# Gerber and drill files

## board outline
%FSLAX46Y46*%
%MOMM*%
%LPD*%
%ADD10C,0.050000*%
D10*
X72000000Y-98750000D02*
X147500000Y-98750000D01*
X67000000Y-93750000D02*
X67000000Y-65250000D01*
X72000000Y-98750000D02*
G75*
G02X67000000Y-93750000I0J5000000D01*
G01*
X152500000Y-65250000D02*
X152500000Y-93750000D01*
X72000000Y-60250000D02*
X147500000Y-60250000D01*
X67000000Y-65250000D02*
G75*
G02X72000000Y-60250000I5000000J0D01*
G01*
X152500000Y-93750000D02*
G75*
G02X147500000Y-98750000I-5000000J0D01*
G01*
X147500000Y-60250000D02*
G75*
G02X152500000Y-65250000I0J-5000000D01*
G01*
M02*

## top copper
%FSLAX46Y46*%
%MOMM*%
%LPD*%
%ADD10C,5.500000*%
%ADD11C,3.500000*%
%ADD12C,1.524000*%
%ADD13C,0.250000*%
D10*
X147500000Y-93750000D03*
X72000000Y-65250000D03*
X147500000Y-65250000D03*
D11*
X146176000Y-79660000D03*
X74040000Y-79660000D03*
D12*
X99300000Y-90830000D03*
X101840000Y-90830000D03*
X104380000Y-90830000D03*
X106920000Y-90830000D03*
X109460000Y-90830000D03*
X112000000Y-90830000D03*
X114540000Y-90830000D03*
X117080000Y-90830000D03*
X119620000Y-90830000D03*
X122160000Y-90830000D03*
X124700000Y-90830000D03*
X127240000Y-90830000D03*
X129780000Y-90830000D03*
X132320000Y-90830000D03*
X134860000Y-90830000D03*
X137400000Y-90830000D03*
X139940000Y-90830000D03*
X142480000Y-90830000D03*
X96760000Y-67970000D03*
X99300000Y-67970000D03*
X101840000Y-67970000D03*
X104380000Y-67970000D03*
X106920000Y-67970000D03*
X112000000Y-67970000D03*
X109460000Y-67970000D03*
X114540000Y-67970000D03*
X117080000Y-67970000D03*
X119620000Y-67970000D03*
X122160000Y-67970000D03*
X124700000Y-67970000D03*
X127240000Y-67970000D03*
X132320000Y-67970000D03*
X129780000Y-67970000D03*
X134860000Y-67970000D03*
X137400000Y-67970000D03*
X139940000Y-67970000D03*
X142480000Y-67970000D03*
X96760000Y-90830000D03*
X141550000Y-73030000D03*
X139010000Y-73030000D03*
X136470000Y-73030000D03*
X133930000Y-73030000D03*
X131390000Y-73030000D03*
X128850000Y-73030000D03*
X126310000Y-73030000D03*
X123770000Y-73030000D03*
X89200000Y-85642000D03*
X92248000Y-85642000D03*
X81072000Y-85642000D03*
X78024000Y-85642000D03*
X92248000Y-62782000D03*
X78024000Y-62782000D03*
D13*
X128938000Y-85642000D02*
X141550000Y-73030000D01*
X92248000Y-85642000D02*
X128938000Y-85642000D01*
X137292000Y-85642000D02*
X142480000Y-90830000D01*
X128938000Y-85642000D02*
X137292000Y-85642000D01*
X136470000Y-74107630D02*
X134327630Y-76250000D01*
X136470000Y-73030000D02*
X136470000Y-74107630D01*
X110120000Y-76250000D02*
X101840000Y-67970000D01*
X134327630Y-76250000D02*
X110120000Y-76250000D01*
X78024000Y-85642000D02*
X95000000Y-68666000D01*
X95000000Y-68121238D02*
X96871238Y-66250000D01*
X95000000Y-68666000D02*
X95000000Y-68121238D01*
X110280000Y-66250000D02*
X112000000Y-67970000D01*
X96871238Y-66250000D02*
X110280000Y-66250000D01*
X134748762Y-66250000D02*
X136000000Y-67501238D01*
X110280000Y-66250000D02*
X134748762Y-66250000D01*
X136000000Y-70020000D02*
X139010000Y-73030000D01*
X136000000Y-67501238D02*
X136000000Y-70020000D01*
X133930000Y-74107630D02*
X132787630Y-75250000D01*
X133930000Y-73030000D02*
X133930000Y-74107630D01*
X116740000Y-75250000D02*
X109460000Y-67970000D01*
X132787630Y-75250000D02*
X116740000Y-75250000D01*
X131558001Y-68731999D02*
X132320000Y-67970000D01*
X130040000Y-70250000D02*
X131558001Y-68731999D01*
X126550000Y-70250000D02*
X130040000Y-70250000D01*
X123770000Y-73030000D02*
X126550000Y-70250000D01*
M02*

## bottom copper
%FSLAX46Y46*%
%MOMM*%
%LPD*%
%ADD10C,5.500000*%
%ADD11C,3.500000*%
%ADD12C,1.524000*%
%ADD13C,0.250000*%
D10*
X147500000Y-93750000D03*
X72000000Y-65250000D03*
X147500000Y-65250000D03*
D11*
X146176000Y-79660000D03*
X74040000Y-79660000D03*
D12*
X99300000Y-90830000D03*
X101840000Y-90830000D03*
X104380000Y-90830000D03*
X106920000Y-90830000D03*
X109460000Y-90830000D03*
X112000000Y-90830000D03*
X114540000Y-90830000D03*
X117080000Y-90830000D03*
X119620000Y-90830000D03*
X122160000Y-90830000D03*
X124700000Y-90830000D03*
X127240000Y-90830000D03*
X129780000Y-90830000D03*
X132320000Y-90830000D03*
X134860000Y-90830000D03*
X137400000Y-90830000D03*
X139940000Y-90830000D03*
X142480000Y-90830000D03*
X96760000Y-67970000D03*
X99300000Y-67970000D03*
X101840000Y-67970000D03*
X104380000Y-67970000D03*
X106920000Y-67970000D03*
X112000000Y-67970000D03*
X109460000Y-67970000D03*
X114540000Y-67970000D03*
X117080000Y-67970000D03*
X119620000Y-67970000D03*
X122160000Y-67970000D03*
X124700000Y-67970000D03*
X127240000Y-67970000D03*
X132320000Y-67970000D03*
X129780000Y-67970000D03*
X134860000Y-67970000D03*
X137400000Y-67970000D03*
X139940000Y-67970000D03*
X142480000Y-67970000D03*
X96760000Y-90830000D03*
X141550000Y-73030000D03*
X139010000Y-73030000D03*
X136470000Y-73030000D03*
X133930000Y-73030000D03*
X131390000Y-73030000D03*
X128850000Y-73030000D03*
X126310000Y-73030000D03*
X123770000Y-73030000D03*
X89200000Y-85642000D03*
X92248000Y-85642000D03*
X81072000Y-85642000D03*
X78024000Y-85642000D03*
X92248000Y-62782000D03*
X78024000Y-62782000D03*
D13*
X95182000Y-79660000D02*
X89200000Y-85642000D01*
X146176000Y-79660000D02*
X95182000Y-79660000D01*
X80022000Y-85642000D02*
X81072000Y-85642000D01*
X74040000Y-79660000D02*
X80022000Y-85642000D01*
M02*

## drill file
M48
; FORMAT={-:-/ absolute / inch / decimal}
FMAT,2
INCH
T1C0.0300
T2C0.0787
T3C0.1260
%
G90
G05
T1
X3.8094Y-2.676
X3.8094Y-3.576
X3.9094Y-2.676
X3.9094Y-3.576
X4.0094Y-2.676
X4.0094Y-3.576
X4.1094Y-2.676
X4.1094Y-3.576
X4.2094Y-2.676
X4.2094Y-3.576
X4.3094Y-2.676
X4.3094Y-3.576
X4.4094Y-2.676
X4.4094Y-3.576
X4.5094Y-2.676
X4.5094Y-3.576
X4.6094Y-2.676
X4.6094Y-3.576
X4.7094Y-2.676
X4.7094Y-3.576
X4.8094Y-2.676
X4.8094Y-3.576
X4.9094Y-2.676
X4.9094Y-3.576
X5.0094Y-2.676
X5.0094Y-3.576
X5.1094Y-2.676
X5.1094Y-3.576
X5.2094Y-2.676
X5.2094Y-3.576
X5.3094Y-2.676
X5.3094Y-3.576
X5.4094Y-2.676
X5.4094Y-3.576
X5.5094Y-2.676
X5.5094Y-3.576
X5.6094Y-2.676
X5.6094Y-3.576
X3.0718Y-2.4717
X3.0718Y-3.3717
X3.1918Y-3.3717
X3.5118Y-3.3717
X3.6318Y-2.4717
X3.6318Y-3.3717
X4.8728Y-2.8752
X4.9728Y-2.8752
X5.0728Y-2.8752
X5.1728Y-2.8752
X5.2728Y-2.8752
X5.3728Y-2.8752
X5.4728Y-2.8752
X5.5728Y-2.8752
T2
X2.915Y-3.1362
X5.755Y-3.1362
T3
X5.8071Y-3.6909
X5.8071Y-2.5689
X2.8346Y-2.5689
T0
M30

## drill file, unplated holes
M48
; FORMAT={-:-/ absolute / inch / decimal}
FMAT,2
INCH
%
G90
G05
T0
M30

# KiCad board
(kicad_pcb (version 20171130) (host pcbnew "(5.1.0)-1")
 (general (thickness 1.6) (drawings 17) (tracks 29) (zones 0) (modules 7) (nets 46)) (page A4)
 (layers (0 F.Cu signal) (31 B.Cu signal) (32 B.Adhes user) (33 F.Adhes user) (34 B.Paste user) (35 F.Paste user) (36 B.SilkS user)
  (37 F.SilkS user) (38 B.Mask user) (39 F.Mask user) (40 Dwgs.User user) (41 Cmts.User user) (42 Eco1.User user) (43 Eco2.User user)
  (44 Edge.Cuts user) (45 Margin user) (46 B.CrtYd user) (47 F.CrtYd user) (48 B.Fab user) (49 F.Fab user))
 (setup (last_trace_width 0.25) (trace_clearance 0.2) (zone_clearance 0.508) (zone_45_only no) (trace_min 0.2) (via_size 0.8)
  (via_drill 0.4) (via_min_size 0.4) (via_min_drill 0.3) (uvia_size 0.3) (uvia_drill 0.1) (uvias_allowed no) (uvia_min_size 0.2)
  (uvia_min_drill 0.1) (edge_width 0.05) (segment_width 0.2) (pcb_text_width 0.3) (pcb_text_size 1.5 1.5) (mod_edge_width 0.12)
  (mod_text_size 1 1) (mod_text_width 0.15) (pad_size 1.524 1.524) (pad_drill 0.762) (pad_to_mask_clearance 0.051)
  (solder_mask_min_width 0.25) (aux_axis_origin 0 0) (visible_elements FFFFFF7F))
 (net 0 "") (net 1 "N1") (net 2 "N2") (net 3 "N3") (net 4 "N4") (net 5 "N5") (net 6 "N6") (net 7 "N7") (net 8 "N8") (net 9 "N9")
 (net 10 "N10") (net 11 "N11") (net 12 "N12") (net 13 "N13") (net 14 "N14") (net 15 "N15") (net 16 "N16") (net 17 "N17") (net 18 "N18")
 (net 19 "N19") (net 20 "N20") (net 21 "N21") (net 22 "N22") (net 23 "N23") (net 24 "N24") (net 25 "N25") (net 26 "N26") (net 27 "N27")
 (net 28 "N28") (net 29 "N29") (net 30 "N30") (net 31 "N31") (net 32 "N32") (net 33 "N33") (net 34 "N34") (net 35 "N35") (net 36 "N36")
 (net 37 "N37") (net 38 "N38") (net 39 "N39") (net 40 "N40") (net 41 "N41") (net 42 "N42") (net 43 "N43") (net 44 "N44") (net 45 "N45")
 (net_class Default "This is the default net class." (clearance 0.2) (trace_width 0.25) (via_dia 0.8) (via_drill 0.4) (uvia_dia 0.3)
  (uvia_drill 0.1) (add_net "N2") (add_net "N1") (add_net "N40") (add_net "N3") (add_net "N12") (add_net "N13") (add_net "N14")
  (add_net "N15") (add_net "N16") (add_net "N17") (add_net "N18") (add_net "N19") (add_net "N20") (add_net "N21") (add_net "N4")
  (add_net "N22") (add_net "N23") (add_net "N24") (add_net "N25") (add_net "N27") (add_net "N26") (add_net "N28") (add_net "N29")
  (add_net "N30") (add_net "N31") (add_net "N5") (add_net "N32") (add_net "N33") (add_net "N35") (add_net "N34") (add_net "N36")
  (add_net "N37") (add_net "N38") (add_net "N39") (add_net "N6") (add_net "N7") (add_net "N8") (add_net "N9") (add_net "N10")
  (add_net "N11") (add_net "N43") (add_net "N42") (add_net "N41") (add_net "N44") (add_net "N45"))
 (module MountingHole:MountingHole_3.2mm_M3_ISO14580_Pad (layer F.Cu) (at 147.5 93.75)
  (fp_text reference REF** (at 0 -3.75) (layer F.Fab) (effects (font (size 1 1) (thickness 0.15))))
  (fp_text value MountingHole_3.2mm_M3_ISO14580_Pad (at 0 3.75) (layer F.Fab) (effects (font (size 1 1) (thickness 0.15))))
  (pad 1 thru_hole circle (at 0 0) (size 5.5 5.5) (drill 3.2) (layers *.Cu *.Mask)))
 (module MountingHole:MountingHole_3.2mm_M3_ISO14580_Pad (layer F.Cu) (at 72 65.25)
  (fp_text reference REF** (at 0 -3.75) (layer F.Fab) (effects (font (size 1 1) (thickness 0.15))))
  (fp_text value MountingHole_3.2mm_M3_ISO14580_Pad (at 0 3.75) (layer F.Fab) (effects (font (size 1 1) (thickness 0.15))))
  (pad 1 thru_hole circle (at 0 0) (size 5.5 5.5) (drill 3.2) (layers *.Cu *.Mask)))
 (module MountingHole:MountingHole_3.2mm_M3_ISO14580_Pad (layer F.Cu) (at 147.5 65.25)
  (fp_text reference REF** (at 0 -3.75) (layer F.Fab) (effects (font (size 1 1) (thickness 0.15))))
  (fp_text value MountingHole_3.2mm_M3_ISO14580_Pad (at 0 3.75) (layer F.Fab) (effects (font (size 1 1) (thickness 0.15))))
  (pad 1 thru_hole circle (at 0 0) (size 5.5 5.5) (drill 3.2) (layers *.Cu *.Mask)))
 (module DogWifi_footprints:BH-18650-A (layer B.Cu) (at 71.5 69.5)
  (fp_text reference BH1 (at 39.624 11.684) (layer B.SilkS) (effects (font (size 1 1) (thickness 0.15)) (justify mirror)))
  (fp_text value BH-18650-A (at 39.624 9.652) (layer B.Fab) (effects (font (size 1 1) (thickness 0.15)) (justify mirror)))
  (pad 1 thru_hole circle (at 74.676 10.16) (size 3.5 3.5) (drill 2) (layers *.Cu *.Mask) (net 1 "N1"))
  (pad 0 thru_hole circle (at 2.54 10.16) (size 3.5 3.5) (drill 2) (layers *.Cu *.Mask) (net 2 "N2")))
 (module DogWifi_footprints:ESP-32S (layer F.Cu) (at 143.75 92.1 90)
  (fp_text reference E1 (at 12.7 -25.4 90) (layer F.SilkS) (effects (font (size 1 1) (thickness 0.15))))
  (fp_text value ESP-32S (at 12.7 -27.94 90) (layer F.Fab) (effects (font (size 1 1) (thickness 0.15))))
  (pad 1 thru_hole circle (at 1.27 -44.45 90) (size 1.524 1.524) (drill 0.762) (layers *.Cu *.Mask) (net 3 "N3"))
  (pad 2 thru_hole circle (at 1.27 -41.91 90) (size 1.524 1.524) (drill 0.762) (layers *.Cu *.Mask) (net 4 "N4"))
  (pad 3 thru_hole circle (at 1.27 -39.37 90) (size 1.524 1.524) (drill 0.762) (layers *.Cu *.Mask) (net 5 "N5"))
  (pad 4 thru_hole circle (at 1.27 -36.83 90) (size 1.524 1.524) (drill 0.762) (layers *.Cu *.Mask) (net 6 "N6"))
  (pad 5 thru_hole circle (at 1.27 -34.29 90) (size 1.524 1.524) (drill 0.762) (layers *.Cu *.Mask) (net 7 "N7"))
  (pad 6 thru_hole circle (at 1.27 -31.75 90) (size 1.524 1.524) (drill 0.762) (layers *.Cu *.Mask) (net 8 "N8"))
  (pad 7 thru_hole circle (at 1.27 -29.21 90) (size 1.524 1.524) (drill 0.762) (layers *.Cu *.Mask) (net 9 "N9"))
  (pad 8 thru_hole circle (at 1.27 -26.67 90) (size 1.524 1.524) (drill 0.762) (layers *.Cu *.Mask) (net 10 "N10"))
  (pad 9 thru_hole circle (at 1.27 -24.13 90) (size 1.524 1.524) (drill 0.762) (layers *.Cu *.Mask) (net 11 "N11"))
  (pad 10 thru_hole circle (at 1.27 -21.59 90) (size 1.524 1.524) (drill 0.762) (layers *.Cu *.Mask) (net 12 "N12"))
  (pad 11 thru_hole circle (at 1.27 -19.05 90) (size 1.524 1.524) (drill 0.762) (layers *.Cu *.Mask) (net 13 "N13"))
  (pad 12 thru_hole circle (at 1.27 -16.51 90) (size 1.524 1.524) (drill 0.762) (layers *.Cu *.Mask) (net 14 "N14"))
  (pad 13 thru_hole circle (at 1.27 -13.97 90) (size 1.524 1.524) (drill 0.762) (layers *.Cu *.Mask) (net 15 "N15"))
  (pad 14 thru_hole circle (at 1.27 -11.43 90) (size 1.524 1.524) (drill 0.762) (layers *.Cu *.Mask) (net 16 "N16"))
  (pad 15 thru_hole circle (at 1.27 -8.89 90) (size 1.524 1.524) (drill 0.762) (layers *.Cu *.Mask) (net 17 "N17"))
  (pad 16 thru_hole circle (at 1.27 -6.35 90) (size 1.524 1.524) (drill 0.762) (layers *.Cu *.Mask) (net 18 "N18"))
  (pad 17 thru_hole circle (at 1.27 -3.81 90) (size 1.524 1.524) (drill 0.762) (layers *.Cu *.Mask) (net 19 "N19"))
  (pad 18 thru_hole circle (at 1.27 -1.27 90) (size 1.524 1.524) (drill 0.762) (layers *.Cu *.Mask) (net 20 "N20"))
  (pad 19 thru_hole circle (at 24.13 -46.99 90) (size 1.524 1.524) (drill 0.762) (layers *.Cu *.Mask) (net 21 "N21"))
  (pad 20 thru_hole circle (at 24.13 -44.45 90) (size 1.524 1.524) (drill 0.762) (layers *.Cu *.Mask) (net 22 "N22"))
  (pad 21 thru_hole circle (at 24.13 -41.91 90) (size 1.524 1.524) (drill 0.762) (layers *.Cu *.Mask) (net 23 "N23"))
  (pad 22 thru_hole circle (at 24.13 -39.37 90) (size 1.524 1.524) (drill 0.762) (layers *.Cu *.Mask) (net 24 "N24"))
  (pad 23 thru_hole circle (at 24.13 -36.83 90) (size 1.524 1.524) (drill 0.762) (layers *.Cu *.Mask) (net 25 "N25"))
  (pad 25 thru_hole circle (at 24.13 -31.75 90) (size 1.524 1.524) (drill 0.762) (layers *.Cu *.Mask) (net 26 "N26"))
  (pad 24 thru_hole circle (at 24.13 -34.29 90) (size 1.524 1.524) (drill 0.762) (layers *.Cu *.Mask) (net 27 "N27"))
  (pad 26 thru_hole circle (at 24.13 -29.21 90) (size 1.524 1.524) (drill 0.762) (layers *.Cu *.Mask) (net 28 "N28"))
  (pad 27 thru_hole circle (at 24.13 -26.67 90) (size 1.524 1.524) (drill 0.762) (layers *.Cu *.Mask) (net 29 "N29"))
  (pad 28 thru_hole circle (at 24.13 -24.13 90) (size 1.524 1.524) (drill 0.762) (layers *.Cu *.Mask) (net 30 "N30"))
  (pad 29 thru_hole circle (at 24.13 -21.59 90) (size 1.524 1.524) (drill 0.762) (layers *.Cu *.Mask) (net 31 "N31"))
  (pad 30 thru_hole circle (at 24.13 -19.05 90) (size 1.524 1.524) (drill 0.762) (layers *.Cu *.Mask) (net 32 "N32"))
  (pad 31 thru_hole circle (at 24.13 -16.51 90) (size 1.524 1.524) (drill 0.762) (layers *.Cu *.Mask) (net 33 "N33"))
  (pad 33 thru_hole circle (at 24.13 -11.43 90) (size 1.524 1.524) (drill 0.762) (layers *.Cu *.Mask) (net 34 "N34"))
  (pad 32 thru_hole circle (at 24.13 -13.97 90) (size 1.524 1.524) (drill 0.762) (layers *.Cu *.Mask) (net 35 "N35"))
  (pad 34 thru_hole circle (at 24.13 -8.89 90) (size 1.524 1.524) (drill 0.762) (layers *.Cu *.Mask) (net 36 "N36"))
  (pad 35 thru_hole circle (at 24.13 -6.35 90) (size 1.524 1.524) (drill 0.762) (layers *.Cu *.Mask) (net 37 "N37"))
  (pad 36 thru_hole circle (at 24.13 -3.81 90) (size 1.524 1.524) (drill 0.762) (layers *.Cu *.Mask) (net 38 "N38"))
  (pad 37 thru_hole circle (at 24.13 -1.27 90) (size 1.524 1.524) (drill 0.762) (layers *.Cu *.Mask) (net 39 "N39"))
  (pad 0 thru_hole circle (at 1.27 -46.99 90) (size 1.524 1.524) (drill 0.762) (layers *.Cu *.Mask) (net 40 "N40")))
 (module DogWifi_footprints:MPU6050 (layer F.Cu) (at 122.5 87)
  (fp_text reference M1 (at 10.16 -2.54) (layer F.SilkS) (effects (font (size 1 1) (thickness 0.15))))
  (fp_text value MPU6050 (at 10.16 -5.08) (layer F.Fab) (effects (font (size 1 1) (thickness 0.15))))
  (pad 7 thru_hole circle (at 19.05 -13.97) (size 1.524 1.524) (drill 0.762) (layers *.Cu *.Mask) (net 20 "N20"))
  (pad 6 thru_hole circle (at 16.51 -13.97) (size 1.524 1.524) (drill 0.762) (layers *.Cu *.Mask) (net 26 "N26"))
  (pad 5 thru_hole circle (at 13.97 -13.97) (size 1.524 1.524) (drill 0.762) (layers *.Cu *.Mask) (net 23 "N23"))
  (pad 4 thru_hole circle (at 11.43 -13.97) (size 1.524 1.524) (drill 0.762) (layers *.Cu *.Mask) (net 27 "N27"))
  (pad 3 thru_hole circle (at 8.89 -13.97) (size 1.524 1.524) (drill 0.762) (layers *.Cu *.Mask) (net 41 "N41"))
  (pad 2 thru_hole circle (at 6.35 -13.97) (size 1.524 1.524) (drill 0.762) (layers *.Cu *.Mask) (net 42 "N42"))
  (pad 1 thru_hole circle (at 3.81 -13.97) (size 1.524 1.524) (drill 0.762) (layers *.Cu *.Mask) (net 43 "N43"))
  (pad 0 thru_hole circle (at 1.27 -13.97) (size 1.524 1.524) (drill 0.762) (layers *.Cu *.Mask) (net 34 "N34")))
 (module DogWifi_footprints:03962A (layer F.Cu) (at 76.5 60.75 270)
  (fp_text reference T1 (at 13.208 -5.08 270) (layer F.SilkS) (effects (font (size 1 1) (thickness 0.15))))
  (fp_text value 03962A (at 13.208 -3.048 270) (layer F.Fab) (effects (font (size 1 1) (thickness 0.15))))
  (pad 3 thru_hole circle (at 24.892 -12.7 270) (size 1.524 1.524) (drill 0.762) (layers *.Cu *.Mask) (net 1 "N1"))
  (pad 2 thru_hole circle (at 24.892 -15.748 270) (size 1.524 1.524) (drill 0.762) (layers *.Cu *.Mask) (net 20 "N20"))
  (pad 4 thru_hole circle (at 24.892 -4.572 270) (size 1.524 1.524) (drill 0.762) (layers *.Cu *.Mask) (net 2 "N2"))
  (pad 5 thru_hole circle (at 24.892 -1.524 270) (size 1.524 1.524) (drill 0.762) (layers *.Cu *.Mask) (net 26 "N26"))
  (pad 0 thru_hole circle (at 2.032 -15.748 270) (size 1.524 1.524) (drill 0.762) (layers *.Cu *.Mask) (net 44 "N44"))
  (pad 1 thru_hole circle (at 2.032 -1.524 270) (size 1.524 1.524) (drill 0.762) (layers *.Cu *.Mask) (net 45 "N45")))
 (gr_line (start 72 98.75) (end 147.5 98.75) (layer Edge.Cuts) (width 0.05))
 (gr_line (start 67 93.75) (end 67 65.25) (layer Edge.Cuts) (width 0.05))
 (gr_arc (start 72 93.75) (end 67 93.75) (angle -90) (layer Edge.Cuts) (width 0.05))
 (gr_line (start 152.5 65.25) (end 152.5 93.75) (layer Edge.Cuts) (width 0.05))
 (gr_line (start 72 60.25) (end 147.5 60.25) (layer Edge.Cuts) (width 0.05))
 (gr_arc (start 72 65.25) (end 72 60.25) (angle -90) (layer Edge.Cuts) (width 0.05))
 (gr_arc (start 147.5 93.75) (end 147.5 98.75) (angle -90) (layer Edge.Cuts) (width 0.05))
 (gr_arc (start 147.5 65.25) (end 152.5 65.25) (angle -90) (layer Edge.Cuts) (width 0.05))
 (segment (start 95.182 79.66) (end 89.2 85.642) (width 0.25) (layer B.Cu) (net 1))
 (segment (start 146.176 79.66) (end 95.182 79.66) (width 0.25) (layer B.Cu) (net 1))
 (segment (start 80.022 85.642) (end 81.072 85.642) (width 0.25) (layer B.Cu) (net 2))
 (segment (start 74.04 79.66) (end 80.022 85.642) (width 0.25) (layer B.Cu) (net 2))
 (segment (start 128.938 85.642) (end 141.55 73.03) (width 0.25) (layer F.Cu) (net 20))
 (segment (start 92.248 85.642) (end 128.938 85.642) (width 0.25) (layer F.Cu) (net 20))
 (segment (start 137.292 85.642) (end 142.48 90.83) (width 0.25) (layer F.Cu) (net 20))
 (segment (start 128.938 85.642) (end 137.292 85.642) (width 0.25) (layer F.Cu) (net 20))
 (segment (start 136.47 74.10763) (end 134.32763 76.25) (width 0.25) (layer F.Cu) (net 23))
 (segment (start 136.47 73.03) (end 136.47 74.10763) (width 0.25) (layer F.Cu) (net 23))
 (segment (start 110.12 76.25) (end 101.84 67.97) (width 0.25) (layer F.Cu) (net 23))
 (segment (start 134.32763 76.25) (end 110.12 76.25) (width 0.25) (layer F.Cu) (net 23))
 (segment (start 78.024 85.642) (end 95 68.666) (width 0.25) (layer F.Cu) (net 26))
 (segment (start 95 68.121238) (end 96.871238 66.25) (width 0.25) (layer F.Cu) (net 26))
 (segment (start 95 68.666) (end 95 68.121238) (width 0.25) (layer F.Cu) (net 26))
 (segment (start 110.28 66.25) (end 112 67.97) (width 0.25) (layer F.Cu) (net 26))
 (segment (start 96.871238 66.25) (end 110.28 66.25) (width 0.25) (layer F.Cu) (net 26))
 (segment (start 134.748762 66.25) (end 136 67.501238) (width 0.25) (layer F.Cu) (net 26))
 (segment (start 110.28 66.25) (end 134.748762 66.25) (width 0.25) (layer F.Cu) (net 26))
 (segment (start 136 70.02) (end 139.01 73.03) (width 0.25) (layer F.Cu) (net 26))
 (segment (start 136 67.501238) (end 136 70.02) (width 0.25) (layer F.Cu) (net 26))
 (segment (start 133.93 74.10763) (end 132.78763 75.25) (width 0.25) (layer F.Cu) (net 27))
 (segment (start 133.93 73.03) (end 133.93 74.10763) (width 0.25) (layer F.Cu) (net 27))
 (segment (start 116.74 75.25) (end 109.46 67.97) (width 0.25) (layer F.Cu) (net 27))
 (segment (start 132.78763 75.25) (end 116.74 75.25) (width 0.25) (layer F.Cu) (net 27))
 (segment (start 131.558001 68.731999) (end 132.32 67.97) (width 0.25) (layer F.Cu) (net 34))
 (segment (start 130.04 70.25) (end 131.558001 68.731999) (width 0.25) (layer F.Cu) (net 34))
 (segment (start 126.55 70.25) (end 130.04 70.25) (width 0.25) (layer F.Cu) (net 34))
 (segment (start 123.77 73.03) (end 126.55 70.25) (width 0.25) (layer F.Cu) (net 34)))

